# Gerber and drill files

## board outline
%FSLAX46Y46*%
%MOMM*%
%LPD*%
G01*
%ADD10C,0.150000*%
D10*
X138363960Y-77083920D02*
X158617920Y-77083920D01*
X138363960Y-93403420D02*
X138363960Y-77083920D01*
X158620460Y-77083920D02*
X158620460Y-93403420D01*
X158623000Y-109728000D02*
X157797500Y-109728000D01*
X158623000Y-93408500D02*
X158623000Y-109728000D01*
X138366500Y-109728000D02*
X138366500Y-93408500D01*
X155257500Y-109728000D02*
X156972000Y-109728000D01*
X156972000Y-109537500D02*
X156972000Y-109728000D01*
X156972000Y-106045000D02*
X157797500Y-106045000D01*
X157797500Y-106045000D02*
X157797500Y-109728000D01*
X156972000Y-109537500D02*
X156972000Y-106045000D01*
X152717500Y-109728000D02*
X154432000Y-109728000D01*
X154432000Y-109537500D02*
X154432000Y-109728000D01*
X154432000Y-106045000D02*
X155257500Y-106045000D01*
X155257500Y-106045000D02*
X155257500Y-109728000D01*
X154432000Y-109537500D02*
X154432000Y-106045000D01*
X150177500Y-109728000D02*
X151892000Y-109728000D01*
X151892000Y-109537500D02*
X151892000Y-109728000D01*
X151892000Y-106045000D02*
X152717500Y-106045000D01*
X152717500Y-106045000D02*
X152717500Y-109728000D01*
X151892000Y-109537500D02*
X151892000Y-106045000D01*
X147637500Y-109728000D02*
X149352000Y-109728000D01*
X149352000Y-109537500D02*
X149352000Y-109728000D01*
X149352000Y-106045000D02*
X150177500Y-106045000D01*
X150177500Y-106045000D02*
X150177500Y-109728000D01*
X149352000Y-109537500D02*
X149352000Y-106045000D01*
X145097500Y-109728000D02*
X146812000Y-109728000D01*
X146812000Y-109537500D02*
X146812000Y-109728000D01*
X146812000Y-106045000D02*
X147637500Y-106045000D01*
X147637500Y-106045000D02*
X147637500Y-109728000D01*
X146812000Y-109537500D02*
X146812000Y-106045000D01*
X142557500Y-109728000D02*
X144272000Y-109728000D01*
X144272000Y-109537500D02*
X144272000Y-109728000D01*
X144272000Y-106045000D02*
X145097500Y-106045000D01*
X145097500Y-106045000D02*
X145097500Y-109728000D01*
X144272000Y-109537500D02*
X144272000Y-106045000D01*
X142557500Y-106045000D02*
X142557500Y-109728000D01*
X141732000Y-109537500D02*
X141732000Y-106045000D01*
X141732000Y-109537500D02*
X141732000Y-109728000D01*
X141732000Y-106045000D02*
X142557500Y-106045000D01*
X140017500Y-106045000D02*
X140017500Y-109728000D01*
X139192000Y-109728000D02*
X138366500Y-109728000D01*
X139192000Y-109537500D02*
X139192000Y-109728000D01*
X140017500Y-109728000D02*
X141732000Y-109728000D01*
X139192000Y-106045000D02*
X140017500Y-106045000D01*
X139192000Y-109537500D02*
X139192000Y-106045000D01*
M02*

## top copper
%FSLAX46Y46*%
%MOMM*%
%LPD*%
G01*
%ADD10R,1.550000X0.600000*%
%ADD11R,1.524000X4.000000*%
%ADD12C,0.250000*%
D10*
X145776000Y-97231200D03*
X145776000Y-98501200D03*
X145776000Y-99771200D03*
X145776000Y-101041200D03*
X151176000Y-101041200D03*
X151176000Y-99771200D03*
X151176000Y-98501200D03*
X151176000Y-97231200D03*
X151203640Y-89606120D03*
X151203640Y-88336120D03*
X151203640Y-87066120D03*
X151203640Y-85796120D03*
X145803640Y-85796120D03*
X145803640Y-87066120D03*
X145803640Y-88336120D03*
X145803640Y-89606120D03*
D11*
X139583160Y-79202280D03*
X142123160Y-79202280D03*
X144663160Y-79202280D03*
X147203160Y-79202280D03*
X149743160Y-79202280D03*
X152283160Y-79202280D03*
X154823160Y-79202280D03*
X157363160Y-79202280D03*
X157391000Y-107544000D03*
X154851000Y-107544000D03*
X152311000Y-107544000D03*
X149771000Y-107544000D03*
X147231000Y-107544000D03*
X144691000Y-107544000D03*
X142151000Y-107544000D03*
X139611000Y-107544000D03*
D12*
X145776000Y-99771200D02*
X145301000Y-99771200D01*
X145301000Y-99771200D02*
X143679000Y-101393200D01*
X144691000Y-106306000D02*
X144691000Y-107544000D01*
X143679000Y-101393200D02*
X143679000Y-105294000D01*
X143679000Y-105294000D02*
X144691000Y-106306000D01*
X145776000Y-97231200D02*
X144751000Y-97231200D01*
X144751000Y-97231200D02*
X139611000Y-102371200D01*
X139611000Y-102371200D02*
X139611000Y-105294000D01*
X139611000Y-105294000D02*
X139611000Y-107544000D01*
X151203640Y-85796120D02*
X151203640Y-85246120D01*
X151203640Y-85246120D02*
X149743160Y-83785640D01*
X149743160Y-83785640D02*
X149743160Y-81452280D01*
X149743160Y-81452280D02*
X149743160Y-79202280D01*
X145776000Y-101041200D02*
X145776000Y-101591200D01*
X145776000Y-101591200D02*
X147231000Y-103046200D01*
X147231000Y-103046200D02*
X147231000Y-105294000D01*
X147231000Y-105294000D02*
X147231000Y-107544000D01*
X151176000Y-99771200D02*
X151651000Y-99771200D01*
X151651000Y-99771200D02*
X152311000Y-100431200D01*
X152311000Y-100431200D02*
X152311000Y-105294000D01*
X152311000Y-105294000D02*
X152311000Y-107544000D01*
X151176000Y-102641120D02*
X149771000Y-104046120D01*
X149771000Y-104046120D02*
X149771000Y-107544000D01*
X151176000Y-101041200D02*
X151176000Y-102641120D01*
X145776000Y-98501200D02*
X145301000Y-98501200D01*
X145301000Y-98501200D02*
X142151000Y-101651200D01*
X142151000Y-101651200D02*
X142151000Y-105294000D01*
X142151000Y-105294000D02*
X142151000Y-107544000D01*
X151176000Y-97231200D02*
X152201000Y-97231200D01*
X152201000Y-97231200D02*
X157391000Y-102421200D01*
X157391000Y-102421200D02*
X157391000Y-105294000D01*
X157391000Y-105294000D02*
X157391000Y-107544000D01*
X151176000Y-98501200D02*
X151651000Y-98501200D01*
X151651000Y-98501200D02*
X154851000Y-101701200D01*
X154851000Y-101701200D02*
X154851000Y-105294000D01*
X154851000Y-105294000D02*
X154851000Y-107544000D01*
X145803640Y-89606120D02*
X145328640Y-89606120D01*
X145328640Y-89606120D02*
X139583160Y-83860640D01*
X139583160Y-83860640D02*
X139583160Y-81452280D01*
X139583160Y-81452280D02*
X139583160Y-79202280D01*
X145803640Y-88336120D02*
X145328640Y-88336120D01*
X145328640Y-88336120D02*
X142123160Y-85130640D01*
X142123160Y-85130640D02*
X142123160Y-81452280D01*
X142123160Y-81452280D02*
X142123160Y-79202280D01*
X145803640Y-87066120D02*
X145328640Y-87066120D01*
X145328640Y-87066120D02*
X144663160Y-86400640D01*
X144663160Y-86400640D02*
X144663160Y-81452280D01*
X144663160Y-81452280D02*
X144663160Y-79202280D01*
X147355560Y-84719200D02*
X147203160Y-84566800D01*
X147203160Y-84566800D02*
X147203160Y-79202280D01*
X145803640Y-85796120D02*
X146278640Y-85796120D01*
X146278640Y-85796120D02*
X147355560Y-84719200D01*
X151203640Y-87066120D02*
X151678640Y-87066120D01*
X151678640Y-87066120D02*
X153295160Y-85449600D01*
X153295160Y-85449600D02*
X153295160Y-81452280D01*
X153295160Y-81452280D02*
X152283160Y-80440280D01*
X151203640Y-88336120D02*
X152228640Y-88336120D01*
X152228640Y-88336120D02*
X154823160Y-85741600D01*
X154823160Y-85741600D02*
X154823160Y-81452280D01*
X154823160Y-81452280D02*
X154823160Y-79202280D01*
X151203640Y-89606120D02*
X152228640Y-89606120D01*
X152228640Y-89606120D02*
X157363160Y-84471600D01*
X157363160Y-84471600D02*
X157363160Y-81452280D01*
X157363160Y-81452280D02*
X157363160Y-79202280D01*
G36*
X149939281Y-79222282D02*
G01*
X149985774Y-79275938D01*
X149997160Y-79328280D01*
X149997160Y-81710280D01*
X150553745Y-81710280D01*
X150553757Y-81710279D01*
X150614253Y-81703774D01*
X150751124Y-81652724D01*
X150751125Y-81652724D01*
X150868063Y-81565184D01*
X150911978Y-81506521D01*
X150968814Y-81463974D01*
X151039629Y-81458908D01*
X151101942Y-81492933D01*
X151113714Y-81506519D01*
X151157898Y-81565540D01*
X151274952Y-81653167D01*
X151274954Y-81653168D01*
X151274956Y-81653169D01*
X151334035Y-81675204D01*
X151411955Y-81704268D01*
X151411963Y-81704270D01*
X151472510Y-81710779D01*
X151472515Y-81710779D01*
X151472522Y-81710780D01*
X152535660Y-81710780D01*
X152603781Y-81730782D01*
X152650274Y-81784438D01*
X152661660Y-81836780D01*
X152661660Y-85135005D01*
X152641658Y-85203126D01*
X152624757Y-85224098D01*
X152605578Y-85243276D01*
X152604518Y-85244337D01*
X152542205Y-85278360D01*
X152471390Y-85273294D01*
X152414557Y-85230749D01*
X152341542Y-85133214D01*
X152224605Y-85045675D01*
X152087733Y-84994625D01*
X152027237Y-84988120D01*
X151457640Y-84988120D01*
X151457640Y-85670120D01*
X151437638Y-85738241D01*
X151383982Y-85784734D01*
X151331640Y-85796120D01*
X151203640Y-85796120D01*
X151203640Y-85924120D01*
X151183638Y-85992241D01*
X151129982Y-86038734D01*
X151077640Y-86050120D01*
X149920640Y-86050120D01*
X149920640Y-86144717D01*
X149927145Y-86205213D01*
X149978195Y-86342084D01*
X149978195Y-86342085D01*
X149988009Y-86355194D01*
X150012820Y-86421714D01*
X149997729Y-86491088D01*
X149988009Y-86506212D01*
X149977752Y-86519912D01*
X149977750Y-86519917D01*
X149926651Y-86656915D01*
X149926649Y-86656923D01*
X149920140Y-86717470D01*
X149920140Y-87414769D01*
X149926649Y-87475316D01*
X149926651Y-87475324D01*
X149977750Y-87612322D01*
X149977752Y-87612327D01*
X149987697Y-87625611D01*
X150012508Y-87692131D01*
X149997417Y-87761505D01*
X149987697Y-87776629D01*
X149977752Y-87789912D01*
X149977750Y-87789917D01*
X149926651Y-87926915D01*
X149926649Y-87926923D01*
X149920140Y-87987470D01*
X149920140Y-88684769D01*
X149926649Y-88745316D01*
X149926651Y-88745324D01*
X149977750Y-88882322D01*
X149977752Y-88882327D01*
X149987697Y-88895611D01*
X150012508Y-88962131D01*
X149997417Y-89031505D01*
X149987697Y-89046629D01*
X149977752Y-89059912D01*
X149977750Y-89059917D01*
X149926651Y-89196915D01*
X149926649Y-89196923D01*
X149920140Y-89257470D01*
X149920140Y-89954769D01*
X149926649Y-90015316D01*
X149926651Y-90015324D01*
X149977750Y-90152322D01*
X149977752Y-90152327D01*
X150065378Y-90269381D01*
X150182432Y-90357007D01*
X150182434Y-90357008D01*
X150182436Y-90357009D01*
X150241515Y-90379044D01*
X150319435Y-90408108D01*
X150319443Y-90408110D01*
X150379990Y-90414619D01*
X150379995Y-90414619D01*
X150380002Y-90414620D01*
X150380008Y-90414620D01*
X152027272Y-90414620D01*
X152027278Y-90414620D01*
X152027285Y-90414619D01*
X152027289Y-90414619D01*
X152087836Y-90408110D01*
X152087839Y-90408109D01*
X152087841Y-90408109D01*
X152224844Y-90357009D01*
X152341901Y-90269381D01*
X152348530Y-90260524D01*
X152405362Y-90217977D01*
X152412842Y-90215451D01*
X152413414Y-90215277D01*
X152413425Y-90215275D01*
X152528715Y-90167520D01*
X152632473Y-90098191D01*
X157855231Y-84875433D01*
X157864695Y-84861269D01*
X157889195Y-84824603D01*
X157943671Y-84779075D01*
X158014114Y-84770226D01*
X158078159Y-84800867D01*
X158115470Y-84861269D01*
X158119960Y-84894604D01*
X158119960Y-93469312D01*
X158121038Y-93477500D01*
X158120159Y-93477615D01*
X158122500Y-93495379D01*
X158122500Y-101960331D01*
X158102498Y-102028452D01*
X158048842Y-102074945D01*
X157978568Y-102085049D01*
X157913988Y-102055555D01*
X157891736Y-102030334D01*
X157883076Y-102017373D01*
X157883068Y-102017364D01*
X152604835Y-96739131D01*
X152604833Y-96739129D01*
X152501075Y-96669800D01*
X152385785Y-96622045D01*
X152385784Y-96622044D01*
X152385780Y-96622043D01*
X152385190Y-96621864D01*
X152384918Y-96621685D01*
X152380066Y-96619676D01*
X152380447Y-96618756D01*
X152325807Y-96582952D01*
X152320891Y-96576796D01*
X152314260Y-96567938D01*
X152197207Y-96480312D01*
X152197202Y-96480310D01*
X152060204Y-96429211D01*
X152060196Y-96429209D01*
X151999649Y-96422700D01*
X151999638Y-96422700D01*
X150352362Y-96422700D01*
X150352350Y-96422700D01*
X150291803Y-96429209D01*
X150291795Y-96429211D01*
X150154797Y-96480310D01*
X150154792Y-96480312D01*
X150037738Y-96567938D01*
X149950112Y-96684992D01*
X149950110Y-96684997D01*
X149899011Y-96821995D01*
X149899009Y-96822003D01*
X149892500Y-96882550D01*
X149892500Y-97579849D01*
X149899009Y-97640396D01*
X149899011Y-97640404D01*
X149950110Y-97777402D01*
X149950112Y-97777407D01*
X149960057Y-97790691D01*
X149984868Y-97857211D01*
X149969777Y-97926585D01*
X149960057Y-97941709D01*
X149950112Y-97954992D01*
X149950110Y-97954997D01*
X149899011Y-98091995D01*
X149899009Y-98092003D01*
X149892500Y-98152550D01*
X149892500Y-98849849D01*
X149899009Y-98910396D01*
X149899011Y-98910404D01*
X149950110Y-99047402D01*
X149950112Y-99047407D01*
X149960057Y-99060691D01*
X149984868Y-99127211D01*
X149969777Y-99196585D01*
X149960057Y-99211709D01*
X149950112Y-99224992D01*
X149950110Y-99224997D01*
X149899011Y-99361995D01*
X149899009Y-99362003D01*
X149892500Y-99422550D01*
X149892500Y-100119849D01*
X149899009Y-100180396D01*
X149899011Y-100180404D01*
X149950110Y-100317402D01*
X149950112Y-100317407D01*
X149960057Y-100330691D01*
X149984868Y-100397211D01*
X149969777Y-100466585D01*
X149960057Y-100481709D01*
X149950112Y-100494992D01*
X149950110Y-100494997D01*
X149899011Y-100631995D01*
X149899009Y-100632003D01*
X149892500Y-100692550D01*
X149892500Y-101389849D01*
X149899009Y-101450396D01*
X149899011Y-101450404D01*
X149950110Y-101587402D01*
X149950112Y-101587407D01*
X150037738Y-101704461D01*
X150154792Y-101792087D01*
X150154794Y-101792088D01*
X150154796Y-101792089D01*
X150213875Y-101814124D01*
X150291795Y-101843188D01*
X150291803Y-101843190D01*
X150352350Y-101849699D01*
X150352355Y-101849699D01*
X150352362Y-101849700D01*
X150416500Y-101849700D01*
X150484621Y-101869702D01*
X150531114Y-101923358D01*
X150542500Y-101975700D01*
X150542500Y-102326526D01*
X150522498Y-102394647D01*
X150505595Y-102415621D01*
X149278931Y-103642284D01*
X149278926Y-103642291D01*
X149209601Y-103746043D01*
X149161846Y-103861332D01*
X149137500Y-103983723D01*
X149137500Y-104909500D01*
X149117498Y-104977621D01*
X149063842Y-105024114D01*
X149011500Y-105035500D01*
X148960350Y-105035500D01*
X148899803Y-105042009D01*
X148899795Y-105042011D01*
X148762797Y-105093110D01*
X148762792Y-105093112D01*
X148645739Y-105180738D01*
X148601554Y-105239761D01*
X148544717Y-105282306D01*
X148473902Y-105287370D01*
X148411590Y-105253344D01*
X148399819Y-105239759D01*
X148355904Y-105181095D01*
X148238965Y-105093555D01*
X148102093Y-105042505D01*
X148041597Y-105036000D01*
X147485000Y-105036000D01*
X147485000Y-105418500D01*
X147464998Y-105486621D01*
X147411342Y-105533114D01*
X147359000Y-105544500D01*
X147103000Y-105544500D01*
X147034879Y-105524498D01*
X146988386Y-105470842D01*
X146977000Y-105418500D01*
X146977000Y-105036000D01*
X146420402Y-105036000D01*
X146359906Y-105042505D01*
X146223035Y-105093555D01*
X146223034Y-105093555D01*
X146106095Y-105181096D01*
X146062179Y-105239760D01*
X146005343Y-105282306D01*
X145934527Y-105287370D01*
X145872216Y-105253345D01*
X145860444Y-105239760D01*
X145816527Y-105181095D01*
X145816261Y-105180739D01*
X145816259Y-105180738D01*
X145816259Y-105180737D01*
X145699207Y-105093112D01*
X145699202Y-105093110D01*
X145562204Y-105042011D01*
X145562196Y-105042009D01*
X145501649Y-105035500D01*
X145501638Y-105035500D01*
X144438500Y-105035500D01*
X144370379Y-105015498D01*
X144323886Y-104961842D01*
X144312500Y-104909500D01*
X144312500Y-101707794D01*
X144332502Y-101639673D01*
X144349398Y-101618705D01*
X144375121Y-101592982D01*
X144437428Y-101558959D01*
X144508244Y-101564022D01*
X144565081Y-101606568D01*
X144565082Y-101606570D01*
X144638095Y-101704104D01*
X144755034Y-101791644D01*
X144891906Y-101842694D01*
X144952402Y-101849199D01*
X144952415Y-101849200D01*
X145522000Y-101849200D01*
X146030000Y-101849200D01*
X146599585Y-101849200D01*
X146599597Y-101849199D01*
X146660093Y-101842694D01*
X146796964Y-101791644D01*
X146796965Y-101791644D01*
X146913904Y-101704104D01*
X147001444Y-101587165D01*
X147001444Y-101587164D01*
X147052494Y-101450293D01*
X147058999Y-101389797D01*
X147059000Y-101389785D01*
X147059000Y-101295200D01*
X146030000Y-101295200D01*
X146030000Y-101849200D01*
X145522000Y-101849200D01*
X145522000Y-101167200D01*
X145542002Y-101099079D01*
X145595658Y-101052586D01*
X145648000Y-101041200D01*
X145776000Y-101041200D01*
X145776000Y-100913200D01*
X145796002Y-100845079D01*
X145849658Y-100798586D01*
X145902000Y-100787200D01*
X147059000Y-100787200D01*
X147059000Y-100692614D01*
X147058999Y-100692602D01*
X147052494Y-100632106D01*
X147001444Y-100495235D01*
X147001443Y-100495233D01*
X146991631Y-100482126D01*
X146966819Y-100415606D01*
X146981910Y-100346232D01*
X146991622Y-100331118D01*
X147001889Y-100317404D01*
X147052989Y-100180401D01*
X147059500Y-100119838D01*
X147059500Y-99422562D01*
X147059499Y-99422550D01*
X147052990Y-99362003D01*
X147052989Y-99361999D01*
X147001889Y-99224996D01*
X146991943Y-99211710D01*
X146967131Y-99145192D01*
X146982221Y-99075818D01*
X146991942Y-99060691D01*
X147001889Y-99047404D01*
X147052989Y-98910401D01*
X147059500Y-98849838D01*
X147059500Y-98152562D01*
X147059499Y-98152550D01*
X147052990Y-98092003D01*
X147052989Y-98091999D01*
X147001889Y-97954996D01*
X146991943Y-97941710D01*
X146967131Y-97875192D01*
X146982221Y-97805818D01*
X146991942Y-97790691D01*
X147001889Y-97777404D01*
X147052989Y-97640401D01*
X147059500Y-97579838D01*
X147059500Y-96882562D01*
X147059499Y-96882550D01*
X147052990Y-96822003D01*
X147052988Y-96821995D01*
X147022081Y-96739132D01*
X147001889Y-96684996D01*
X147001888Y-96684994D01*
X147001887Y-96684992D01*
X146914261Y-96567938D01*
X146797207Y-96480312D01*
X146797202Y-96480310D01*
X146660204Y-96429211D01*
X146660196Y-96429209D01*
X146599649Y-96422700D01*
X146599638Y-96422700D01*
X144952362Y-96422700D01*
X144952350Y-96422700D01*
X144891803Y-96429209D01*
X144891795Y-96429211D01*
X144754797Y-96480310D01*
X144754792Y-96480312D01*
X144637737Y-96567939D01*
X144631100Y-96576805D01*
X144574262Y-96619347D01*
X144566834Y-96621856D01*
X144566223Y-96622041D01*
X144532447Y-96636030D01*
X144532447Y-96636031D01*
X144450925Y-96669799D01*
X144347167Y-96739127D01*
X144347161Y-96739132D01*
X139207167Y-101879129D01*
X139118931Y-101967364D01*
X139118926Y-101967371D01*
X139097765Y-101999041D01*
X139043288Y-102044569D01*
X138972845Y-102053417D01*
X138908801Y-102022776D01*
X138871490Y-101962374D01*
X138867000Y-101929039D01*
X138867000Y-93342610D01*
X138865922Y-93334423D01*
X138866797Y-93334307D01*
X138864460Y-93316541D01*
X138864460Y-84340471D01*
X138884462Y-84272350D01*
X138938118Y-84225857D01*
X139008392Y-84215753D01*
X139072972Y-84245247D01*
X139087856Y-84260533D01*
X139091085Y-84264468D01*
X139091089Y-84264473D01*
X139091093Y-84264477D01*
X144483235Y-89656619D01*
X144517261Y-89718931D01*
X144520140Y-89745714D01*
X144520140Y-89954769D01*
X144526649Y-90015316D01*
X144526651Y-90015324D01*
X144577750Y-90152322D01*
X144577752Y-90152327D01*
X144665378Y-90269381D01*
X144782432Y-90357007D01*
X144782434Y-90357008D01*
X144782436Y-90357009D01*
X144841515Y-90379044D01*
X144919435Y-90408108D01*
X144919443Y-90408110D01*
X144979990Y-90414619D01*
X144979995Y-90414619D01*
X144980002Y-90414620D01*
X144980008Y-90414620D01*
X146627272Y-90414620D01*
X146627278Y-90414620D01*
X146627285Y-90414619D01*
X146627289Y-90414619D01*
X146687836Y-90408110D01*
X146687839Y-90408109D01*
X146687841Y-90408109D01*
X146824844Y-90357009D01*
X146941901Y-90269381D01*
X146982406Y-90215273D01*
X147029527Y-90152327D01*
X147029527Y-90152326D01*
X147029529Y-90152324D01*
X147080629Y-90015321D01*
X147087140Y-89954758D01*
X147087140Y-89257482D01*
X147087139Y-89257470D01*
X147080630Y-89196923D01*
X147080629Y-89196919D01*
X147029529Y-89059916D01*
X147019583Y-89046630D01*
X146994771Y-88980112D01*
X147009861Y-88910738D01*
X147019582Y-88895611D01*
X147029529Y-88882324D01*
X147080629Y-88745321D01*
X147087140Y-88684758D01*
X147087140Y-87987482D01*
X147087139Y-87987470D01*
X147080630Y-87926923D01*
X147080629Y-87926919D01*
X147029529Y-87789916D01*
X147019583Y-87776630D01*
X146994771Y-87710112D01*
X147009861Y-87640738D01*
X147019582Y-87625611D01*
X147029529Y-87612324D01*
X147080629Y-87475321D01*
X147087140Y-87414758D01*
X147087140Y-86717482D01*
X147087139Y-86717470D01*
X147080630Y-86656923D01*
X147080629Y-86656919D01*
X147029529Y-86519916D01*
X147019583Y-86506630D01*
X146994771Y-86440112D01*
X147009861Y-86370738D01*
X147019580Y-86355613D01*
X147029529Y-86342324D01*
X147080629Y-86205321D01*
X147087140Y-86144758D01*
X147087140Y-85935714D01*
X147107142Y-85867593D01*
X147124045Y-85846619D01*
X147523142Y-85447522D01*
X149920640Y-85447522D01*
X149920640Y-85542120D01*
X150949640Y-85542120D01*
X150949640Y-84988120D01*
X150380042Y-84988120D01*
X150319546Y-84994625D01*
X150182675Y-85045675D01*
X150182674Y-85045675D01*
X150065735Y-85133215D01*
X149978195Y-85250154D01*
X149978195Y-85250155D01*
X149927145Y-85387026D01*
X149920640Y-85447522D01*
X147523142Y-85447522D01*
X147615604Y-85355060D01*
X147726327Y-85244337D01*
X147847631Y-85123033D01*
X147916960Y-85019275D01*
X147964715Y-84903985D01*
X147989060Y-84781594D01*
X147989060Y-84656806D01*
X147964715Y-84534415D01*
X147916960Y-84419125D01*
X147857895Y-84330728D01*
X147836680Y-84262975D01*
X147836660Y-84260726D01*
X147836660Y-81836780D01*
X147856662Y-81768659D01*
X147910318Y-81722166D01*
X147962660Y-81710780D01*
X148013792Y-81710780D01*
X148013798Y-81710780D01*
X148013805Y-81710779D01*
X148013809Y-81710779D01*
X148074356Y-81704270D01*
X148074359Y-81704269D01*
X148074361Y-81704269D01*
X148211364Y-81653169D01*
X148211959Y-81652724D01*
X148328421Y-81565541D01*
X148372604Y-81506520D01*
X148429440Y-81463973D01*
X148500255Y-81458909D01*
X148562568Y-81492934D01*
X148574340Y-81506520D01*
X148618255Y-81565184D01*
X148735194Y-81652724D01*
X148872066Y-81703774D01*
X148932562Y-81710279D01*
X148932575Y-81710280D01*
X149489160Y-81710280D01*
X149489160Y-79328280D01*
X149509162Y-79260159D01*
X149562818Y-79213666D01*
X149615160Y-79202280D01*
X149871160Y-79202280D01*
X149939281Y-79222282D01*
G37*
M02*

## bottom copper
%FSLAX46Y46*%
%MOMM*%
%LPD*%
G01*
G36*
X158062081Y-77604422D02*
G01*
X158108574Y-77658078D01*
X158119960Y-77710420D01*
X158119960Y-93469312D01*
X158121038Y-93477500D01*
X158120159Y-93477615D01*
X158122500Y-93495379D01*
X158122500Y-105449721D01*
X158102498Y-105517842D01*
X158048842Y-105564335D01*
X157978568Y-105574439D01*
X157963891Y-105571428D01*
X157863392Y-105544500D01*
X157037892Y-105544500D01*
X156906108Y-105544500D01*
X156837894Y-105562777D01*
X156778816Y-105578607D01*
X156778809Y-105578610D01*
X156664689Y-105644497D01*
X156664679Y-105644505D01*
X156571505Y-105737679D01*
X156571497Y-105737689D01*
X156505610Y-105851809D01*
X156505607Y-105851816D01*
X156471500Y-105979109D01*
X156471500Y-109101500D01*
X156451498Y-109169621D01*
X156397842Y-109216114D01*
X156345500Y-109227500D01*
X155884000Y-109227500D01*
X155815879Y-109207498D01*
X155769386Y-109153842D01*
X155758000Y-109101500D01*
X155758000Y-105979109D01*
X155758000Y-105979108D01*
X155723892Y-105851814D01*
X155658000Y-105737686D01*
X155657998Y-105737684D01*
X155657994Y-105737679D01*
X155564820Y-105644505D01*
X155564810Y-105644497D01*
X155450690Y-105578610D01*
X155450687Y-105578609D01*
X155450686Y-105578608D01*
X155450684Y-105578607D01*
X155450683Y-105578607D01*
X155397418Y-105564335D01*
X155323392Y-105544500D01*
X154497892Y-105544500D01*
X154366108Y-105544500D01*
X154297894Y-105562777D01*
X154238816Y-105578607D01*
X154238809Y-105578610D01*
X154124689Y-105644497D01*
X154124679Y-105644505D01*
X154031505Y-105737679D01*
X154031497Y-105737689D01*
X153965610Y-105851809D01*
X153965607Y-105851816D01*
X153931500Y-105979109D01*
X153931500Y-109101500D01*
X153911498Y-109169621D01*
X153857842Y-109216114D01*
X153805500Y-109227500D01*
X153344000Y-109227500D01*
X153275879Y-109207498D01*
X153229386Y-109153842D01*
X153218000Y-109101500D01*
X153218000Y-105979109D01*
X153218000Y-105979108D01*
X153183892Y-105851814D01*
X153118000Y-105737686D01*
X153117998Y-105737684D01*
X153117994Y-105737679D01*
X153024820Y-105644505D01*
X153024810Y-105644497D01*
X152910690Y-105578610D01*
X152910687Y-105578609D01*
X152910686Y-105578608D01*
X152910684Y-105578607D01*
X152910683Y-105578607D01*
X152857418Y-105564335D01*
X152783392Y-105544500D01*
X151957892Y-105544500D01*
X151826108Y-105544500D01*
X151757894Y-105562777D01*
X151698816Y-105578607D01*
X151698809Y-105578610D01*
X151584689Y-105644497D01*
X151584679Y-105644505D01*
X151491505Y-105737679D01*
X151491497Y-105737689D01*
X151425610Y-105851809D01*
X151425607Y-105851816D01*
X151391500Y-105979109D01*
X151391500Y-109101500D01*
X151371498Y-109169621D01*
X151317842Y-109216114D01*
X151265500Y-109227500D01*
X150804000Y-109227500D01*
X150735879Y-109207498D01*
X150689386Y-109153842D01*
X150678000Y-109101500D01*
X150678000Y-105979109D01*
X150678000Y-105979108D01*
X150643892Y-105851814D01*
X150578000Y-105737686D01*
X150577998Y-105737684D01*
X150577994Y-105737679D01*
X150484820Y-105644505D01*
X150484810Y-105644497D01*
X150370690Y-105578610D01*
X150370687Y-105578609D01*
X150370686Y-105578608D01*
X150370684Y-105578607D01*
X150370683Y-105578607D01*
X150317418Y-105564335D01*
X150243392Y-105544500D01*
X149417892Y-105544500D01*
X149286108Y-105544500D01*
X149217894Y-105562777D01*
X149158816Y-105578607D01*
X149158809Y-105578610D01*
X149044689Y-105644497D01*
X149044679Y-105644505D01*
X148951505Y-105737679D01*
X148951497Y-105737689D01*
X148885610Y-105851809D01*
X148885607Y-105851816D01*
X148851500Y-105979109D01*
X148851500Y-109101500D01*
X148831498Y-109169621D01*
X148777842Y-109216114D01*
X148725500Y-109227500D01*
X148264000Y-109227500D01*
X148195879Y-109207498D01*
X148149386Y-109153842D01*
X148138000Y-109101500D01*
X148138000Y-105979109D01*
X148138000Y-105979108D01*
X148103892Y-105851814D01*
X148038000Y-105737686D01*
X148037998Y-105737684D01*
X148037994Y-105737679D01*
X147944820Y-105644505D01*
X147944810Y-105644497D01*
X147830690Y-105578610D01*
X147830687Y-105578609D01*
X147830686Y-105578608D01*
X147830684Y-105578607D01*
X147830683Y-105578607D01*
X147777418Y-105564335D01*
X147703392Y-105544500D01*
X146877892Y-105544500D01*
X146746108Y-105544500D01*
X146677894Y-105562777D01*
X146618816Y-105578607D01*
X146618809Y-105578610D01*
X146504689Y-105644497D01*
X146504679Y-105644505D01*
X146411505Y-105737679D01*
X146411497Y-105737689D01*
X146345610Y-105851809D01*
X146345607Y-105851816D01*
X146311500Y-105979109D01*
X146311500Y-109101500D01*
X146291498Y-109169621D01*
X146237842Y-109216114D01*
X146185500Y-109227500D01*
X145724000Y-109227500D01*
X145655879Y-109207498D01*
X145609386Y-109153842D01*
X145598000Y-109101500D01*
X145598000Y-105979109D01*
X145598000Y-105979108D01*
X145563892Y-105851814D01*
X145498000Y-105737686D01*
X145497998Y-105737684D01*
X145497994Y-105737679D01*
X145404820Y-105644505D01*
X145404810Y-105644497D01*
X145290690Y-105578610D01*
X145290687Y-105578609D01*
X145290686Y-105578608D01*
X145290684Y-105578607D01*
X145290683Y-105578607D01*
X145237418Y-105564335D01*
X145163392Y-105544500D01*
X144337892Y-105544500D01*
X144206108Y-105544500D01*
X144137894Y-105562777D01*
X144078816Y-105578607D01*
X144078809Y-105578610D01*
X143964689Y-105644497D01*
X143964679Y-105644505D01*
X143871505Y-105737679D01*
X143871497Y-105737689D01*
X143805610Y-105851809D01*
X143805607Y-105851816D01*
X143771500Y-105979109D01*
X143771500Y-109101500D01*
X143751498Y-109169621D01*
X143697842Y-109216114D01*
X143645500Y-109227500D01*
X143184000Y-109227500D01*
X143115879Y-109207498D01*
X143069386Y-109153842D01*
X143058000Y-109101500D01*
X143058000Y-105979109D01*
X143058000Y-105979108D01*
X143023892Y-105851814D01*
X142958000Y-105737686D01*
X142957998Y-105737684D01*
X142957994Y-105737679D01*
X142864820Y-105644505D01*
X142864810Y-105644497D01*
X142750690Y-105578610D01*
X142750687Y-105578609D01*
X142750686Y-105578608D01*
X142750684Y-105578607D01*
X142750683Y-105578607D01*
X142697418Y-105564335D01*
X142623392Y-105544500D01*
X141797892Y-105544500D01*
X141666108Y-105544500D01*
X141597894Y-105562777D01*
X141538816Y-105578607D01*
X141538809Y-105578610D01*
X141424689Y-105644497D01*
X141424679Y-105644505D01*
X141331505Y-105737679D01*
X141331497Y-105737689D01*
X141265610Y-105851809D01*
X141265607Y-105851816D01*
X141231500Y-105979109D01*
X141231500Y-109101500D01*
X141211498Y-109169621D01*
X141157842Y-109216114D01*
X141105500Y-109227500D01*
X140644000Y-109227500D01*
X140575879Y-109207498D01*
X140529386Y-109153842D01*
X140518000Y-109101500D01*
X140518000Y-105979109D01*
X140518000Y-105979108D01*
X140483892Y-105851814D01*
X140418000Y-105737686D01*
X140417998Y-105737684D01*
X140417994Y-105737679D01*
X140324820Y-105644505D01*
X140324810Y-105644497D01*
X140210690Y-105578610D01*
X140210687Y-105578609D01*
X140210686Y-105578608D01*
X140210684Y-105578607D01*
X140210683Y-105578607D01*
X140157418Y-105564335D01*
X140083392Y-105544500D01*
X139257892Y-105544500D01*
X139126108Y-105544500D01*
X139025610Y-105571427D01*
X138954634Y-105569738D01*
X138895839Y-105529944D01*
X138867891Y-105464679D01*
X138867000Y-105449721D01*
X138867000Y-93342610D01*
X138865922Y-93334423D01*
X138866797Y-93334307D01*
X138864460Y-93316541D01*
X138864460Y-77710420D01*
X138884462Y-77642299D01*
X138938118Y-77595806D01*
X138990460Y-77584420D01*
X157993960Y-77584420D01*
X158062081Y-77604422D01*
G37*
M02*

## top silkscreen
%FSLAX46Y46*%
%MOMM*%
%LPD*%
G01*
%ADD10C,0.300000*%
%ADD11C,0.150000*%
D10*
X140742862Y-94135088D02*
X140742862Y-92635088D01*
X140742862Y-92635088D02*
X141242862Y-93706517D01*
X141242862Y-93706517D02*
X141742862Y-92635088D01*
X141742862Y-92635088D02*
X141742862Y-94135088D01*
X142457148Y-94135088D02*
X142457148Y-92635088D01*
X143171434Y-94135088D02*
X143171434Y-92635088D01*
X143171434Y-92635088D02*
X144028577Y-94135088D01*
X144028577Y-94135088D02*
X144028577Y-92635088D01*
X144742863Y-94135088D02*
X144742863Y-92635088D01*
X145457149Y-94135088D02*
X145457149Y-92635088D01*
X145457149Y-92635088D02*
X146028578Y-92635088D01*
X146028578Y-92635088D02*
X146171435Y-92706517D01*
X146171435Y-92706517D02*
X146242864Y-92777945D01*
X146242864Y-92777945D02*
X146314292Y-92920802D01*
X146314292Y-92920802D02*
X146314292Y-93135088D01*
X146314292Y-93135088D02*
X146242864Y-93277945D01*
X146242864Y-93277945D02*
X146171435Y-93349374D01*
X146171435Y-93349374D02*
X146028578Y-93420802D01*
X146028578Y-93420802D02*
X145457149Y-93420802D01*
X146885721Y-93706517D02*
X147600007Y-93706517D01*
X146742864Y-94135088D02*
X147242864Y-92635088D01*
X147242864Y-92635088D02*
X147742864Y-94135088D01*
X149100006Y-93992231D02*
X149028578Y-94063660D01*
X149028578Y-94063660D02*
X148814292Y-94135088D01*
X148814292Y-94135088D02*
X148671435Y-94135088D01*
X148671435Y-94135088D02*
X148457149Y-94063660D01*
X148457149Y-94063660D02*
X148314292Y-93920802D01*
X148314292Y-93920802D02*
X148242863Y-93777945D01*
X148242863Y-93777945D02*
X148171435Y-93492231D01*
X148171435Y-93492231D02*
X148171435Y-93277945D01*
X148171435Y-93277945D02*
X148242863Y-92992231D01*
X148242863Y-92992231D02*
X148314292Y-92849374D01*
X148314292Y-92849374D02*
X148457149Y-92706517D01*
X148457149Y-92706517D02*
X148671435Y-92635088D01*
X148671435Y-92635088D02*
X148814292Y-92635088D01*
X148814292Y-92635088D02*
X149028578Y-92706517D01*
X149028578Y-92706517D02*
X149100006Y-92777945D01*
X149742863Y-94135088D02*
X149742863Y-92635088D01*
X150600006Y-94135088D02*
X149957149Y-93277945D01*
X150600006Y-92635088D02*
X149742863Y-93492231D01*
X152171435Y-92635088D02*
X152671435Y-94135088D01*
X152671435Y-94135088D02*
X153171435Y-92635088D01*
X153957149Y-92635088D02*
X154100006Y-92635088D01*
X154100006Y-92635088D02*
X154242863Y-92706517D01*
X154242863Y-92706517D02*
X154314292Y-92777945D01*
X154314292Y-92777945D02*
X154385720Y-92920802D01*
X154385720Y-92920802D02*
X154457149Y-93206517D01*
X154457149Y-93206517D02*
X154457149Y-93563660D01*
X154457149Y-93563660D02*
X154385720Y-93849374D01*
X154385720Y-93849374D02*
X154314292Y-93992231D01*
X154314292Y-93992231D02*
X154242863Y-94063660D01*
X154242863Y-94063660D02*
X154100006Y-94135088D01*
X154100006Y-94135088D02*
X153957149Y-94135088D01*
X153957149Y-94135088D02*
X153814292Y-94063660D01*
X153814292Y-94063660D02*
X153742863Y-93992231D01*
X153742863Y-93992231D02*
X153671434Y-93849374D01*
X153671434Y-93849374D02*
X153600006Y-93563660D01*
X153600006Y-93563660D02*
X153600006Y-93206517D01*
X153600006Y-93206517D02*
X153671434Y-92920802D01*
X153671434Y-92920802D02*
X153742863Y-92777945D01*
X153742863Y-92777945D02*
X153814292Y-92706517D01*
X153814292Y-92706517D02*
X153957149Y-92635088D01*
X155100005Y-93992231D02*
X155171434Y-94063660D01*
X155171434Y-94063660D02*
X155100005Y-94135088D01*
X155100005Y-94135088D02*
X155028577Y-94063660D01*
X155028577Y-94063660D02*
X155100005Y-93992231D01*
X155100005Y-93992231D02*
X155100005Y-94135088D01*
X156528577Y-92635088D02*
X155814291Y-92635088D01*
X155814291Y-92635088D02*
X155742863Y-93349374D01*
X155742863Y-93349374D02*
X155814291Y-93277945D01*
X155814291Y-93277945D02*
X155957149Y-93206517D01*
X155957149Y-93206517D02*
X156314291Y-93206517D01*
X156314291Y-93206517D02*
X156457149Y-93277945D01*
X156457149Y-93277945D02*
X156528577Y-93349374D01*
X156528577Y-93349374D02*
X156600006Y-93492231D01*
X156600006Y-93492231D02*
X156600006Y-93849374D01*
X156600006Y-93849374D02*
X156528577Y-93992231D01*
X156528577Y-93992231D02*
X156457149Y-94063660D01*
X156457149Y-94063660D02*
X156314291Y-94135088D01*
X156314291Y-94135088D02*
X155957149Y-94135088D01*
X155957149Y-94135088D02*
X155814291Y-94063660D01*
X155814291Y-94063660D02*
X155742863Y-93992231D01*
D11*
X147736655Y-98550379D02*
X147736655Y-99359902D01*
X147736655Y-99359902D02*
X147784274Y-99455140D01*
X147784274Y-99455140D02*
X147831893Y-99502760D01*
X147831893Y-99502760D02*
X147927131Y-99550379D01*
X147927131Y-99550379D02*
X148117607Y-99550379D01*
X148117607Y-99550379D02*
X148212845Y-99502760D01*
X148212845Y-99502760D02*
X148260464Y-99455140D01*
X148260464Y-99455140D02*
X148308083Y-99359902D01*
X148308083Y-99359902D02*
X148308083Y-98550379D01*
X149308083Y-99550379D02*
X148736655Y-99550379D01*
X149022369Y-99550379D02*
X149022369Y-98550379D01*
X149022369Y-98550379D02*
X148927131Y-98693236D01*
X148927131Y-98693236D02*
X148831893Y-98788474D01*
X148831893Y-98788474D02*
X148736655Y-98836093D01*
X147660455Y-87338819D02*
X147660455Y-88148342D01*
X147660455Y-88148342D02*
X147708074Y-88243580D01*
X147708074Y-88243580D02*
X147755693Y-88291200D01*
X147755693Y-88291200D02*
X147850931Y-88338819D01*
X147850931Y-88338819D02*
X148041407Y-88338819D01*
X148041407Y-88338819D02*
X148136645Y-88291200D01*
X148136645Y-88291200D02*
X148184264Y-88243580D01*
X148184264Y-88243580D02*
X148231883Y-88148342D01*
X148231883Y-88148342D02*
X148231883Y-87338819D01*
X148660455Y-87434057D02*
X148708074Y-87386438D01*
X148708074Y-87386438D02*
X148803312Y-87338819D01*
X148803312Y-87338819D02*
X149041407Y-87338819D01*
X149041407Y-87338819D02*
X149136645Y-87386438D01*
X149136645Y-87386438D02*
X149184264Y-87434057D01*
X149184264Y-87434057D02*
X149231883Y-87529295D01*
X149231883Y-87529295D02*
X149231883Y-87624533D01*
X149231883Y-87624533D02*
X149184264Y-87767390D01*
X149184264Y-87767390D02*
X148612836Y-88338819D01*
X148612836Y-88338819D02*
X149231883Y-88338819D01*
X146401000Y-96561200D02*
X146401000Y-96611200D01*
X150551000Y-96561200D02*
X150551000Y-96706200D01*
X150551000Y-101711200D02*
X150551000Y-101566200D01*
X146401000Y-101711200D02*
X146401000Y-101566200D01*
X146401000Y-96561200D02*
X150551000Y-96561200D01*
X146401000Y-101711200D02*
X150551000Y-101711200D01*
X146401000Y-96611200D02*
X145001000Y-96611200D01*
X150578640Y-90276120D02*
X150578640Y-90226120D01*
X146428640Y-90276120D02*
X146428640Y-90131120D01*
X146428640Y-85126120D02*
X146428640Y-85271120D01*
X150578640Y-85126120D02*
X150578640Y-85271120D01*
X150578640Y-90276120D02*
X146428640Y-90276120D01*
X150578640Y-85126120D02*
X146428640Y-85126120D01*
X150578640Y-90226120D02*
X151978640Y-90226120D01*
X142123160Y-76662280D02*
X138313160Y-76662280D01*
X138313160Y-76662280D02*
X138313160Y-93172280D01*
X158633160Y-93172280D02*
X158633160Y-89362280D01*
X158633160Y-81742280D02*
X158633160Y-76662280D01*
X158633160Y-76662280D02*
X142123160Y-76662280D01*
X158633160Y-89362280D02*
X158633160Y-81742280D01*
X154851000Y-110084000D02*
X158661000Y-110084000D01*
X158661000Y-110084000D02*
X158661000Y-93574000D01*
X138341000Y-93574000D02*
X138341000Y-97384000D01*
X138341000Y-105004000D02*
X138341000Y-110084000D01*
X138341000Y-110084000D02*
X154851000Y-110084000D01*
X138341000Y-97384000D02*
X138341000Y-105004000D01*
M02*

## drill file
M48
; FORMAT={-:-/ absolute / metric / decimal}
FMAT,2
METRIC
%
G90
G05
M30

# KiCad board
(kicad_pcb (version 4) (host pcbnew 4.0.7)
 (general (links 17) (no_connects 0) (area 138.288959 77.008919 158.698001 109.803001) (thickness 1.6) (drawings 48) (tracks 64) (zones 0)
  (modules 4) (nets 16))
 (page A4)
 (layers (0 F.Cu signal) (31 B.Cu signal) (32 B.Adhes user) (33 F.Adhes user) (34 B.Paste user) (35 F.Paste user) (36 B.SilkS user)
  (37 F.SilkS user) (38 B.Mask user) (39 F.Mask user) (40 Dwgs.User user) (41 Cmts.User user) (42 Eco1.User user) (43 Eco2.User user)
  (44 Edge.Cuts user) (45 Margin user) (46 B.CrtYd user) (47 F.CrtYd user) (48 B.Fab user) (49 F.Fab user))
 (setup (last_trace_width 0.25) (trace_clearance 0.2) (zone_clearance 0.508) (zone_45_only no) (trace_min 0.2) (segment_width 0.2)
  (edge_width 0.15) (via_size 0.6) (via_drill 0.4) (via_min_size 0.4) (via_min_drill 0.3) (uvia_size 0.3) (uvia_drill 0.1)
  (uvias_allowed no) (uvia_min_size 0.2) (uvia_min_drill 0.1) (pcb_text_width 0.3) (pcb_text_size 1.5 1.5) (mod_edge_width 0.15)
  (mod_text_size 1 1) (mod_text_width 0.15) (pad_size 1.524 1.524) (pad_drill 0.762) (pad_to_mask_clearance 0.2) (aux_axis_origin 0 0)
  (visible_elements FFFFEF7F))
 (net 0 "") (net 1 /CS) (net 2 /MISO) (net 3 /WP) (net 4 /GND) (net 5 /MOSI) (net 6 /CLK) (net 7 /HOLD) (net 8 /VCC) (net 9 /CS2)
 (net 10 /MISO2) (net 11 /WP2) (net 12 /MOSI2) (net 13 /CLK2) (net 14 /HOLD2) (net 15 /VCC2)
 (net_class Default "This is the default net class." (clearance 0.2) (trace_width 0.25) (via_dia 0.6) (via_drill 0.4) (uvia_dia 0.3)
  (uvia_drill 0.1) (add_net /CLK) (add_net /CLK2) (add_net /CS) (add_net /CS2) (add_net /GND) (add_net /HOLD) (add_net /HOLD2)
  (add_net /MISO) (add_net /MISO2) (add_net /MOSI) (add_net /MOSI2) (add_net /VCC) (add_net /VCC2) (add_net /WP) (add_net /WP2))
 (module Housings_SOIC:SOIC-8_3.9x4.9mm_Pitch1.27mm (layer F.Cu) (at 148.476 99.1362)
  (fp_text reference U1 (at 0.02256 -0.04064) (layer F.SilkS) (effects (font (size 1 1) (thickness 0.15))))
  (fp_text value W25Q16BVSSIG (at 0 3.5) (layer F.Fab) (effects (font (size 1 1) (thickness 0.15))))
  (fp_line (start -2.075 -2.575) (end -2.075 -2.525) (layer F.SilkS) (width 0.15))
  (fp_line (start 2.075 -2.575) (end 2.075 -2.43) (layer F.SilkS) (width 0.15))
  (fp_line (start 2.075 2.575) (end 2.075 2.43) (layer F.SilkS) (width 0.15))
  (fp_line (start -2.075 2.575) (end -2.075 2.43) (layer F.SilkS) (width 0.15))
  (fp_line (start -2.075 -2.575) (end 2.075 -2.575) (layer F.SilkS) (width 0.15))
  (fp_line (start -2.075 2.575) (end 2.075 2.575) (layer F.SilkS) (width 0.15))
  (fp_line (start -2.075 -2.525) (end -3.475 -2.525) (layer F.SilkS) (width 0.15))
  (pad 1 smd rect (at -2.7 -1.905) (size 1.55 0.6) (layers F.Cu F.Paste F.Mask) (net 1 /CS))
  (pad 2 smd rect (at -2.7 -0.635) (size 1.55 0.6) (layers F.Cu F.Paste F.Mask) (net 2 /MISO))
  (pad 3 smd rect (at -2.7 0.635) (size 1.55 0.6) (layers F.Cu F.Paste F.Mask) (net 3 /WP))
  (pad 4 smd rect (at -2.7 1.905) (size 1.55 0.6) (layers F.Cu F.Paste F.Mask) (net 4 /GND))
  (pad 5 smd rect (at 2.7 1.905) (size 1.55 0.6) (layers F.Cu F.Paste F.Mask) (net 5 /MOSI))
  (pad 6 smd rect (at 2.7 0.635) (size 1.55 0.6) (layers F.Cu F.Paste F.Mask) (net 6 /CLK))
  (pad 7 smd rect (at 2.7 -0.635) (size 1.55 0.6) (layers F.Cu F.Paste F.Mask) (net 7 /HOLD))
  (pad 8 smd rect (at 2.7 -1.905) (size 1.55 0.6) (layers F.Cu F.Paste F.Mask) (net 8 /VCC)))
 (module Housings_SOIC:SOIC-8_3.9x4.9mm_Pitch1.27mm (layer F.Cu) (at 148.50364 87.70112 180)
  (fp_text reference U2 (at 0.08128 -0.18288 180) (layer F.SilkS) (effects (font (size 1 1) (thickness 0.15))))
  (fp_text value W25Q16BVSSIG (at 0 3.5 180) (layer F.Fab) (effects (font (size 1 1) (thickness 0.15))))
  (fp_line (start -2.075 -2.575) (end -2.075 -2.525) (layer F.SilkS) (width 0.15))
  (fp_line (start 2.075 -2.575) (end 2.075 -2.43) (layer F.SilkS) (width 0.15))
  (fp_line (start 2.075 2.575) (end 2.075 2.43) (layer F.SilkS) (width 0.15))
  (fp_line (start -2.075 2.575) (end -2.075 2.43) (layer F.SilkS) (width 0.15))
  (fp_line (start -2.075 -2.575) (end 2.075 -2.575) (layer F.SilkS) (width 0.15))
  (fp_line (start -2.075 2.575) (end 2.075 2.575) (layer F.SilkS) (width 0.15))
  (fp_line (start -2.075 -2.525) (end -3.475 -2.525) (layer F.SilkS) (width 0.15))
  (pad 1 smd rect (at -2.7 -1.905 180) (size 1.55 0.6) (layers F.Cu F.Paste F.Mask) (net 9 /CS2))
  (pad 2 smd rect (at -2.7 -0.635 180) (size 1.55 0.6) (layers F.Cu F.Paste F.Mask) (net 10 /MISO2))
  (pad 3 smd rect (at -2.7 0.635 180) (size 1.55 0.6) (layers F.Cu F.Paste F.Mask) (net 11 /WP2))
  (pad 4 smd rect (at -2.7 1.905 180) (size 1.55 0.6) (layers F.Cu F.Paste F.Mask) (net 4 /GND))
  (pad 5 smd rect (at 2.7 1.905 180) (size 1.55 0.6) (layers F.Cu F.Paste F.Mask) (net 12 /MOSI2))
  (pad 6 smd rect (at 2.7 0.635 180) (size 1.55 0.6) (layers F.Cu F.Paste F.Mask) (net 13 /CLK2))
  (pad 7 smd rect (at 2.7 -0.635 180) (size 1.55 0.6) (layers F.Cu F.Paste F.Mask) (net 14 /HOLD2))
  (pad 8 smd rect (at 2.7 -1.905 180) (size 1.55 0.6) (layers F.Cu F.Paste F.Mask) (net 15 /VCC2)))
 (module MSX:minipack (layer F.Cu) (at 148.47316 81.74228 180)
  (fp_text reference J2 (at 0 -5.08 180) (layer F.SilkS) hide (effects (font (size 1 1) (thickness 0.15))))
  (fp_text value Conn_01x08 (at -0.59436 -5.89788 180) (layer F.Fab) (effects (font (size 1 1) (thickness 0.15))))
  (fp_line (start 6.35 5.08) (end 10.16 5.08) (layer F.SilkS) (width 0.15))
  (fp_line (start 10.16 5.08) (end 10.16 -11.43) (layer F.SilkS) (width 0.15))
  (fp_line (start -10.16 -11.43) (end -10.16 -7.62) (layer F.SilkS) (width 0.15))
  (fp_line (start -10.16 0) (end -10.16 5.08) (layer F.SilkS) (width 0.15))
  (fp_line (start -10.16 5.08) (end 6.35 5.08) (layer F.SilkS) (width 0.15))
  (fp_line (start -10.16 -7.62) (end -10.16 0) (layer F.SilkS) (width 0.15))
  (pad 8 smd rect (at 8.89 2.54 180) (size 1.524 4) (layers F.Cu F.Paste F.Mask) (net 15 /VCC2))
  (pad 7 smd rect (at 6.35 2.54 180) (size 1.524 4) (layers F.Cu F.Paste F.Mask) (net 14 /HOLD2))
  (pad 6 smd rect (at 3.81 2.54 180) (size 1.524 4) (layers F.Cu F.Paste F.Mask) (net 13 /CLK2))
  (pad 5 smd rect (at 1.27 2.54 180) (size 1.524 4) (layers F.Cu F.Paste F.Mask) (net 12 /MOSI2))
  (pad 4 smd rect (at -1.27 2.54 180) (size 1.524 4) (layers F.Cu F.Paste F.Mask) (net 4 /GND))
  (pad 3 smd rect (at -3.81 2.54 180) (size 1.524 4) (layers F.Cu F.Paste F.Mask) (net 11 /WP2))
  (pad 2 smd rect (at -6.35 2.54 180) (size 1.524 4) (layers F.Cu F.Paste F.Mask) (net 10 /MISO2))
  (pad 1 smd rect (at -8.89 2.54 180) (size 1.524 4) (layers F.Cu F.Paste F.Mask) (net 9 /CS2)))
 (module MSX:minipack (layer F.Cu) (at 148.501 105.004)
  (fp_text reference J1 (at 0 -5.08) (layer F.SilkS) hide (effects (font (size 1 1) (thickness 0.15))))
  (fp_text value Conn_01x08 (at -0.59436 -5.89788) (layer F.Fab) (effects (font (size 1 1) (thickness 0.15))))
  (fp_line (start 6.35 5.08) (end 10.16 5.08) (layer F.SilkS) (width 0.15))
  (fp_line (start 10.16 5.08) (end 10.16 -11.43) (layer F.SilkS) (width 0.15))
  (fp_line (start -10.16 -11.43) (end -10.16 -7.62) (layer F.SilkS) (width 0.15))
  (fp_line (start -10.16 0) (end -10.16 5.08) (layer F.SilkS) (width 0.15))
  (fp_line (start -10.16 5.08) (end 6.35 5.08) (layer F.SilkS) (width 0.15))
  (fp_line (start -10.16 -7.62) (end -10.16 0) (layer F.SilkS) (width 0.15))
  (pad 8 smd rect (at 8.89 2.54) (size 1.524 4) (layers F.Cu F.Paste F.Mask) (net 8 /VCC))
  (pad 7 smd rect (at 6.35 2.54) (size 1.524 4) (layers F.Cu F.Paste F.Mask) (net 7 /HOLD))
  (pad 6 smd rect (at 3.81 2.54) (size 1.524 4) (layers F.Cu F.Paste F.Mask) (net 6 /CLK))
  (pad 5 smd rect (at 1.27 2.54) (size 1.524 4) (layers F.Cu F.Paste F.Mask) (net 5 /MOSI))
  (pad 4 smd rect (at -1.27 2.54) (size 1.524 4) (layers F.Cu F.Paste F.Mask) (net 4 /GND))
  (pad 3 smd rect (at -3.81 2.54) (size 1.524 4) (layers F.Cu F.Paste F.Mask) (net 3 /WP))
  (pad 2 smd rect (at -6.35 2.54) (size 1.524 4) (layers F.Cu F.Paste F.Mask) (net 2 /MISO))
  (pad 1 smd rect (at -8.89 2.54) (size 1.524 4) (layers F.Cu F.Paste F.Mask) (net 1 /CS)))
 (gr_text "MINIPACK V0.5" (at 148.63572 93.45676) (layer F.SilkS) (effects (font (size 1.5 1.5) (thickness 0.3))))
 (gr_line (start 138.36396 77.08392) (end 158.61792 77.08392) (layer Edge.Cuts) (width 0.15))
 (gr_line (start 138.36396 93.40342) (end 138.36396 77.08392) (layer Edge.Cuts) (width 0.15))
 (gr_line (start 158.62046 77.08392) (end 158.62046 93.40342) (layer Edge.Cuts) (width 0.15))
 (gr_line (start 158.623 109.728) (end 157.7975 109.728) (layer Edge.Cuts) (width 0.15))
 (gr_line (start 158.623 93.4085) (end 158.623 109.728) (layer Edge.Cuts) (width 0.15))
 (gr_line (start 138.3665 109.728) (end 138.3665 93.4085) (layer Edge.Cuts) (width 0.15))
 (gr_line (start 155.2575 109.728) (end 156.972 109.728) (layer Edge.Cuts) (width 0.15))
 (gr_line (start 156.972 109.5375) (end 156.972 109.728) (layer Edge.Cuts) (width 0.15))
 (gr_line (start 156.972 106.045) (end 157.7975 106.045) (layer Edge.Cuts) (width 0.15))
 (gr_line (start 157.7975 106.045) (end 157.7975 109.728) (layer Edge.Cuts) (width 0.15))
 (gr_line (start 156.972 109.5375) (end 156.972 106.045) (layer Edge.Cuts) (width 0.15))
 (gr_line (start 152.7175 109.728) (end 154.432 109.728) (layer Edge.Cuts) (width 0.15))
 (gr_line (start 154.432 109.5375) (end 154.432 109.728) (layer Edge.Cuts) (width 0.15))
 (gr_line (start 154.432 106.045) (end 155.2575 106.045) (layer Edge.Cuts) (width 0.15))
 (gr_line (start 155.2575 106.045) (end 155.2575 109.728) (layer Edge.Cuts) (width 0.15))
 (gr_line (start 154.432 109.5375) (end 154.432 106.045) (layer Edge.Cuts) (width 0.15))
 (gr_line (start 150.1775 109.728) (end 151.892 109.728) (layer Edge.Cuts) (width 0.15))
 (gr_line (start 151.892 109.5375) (end 151.892 109.728) (layer Edge.Cuts) (width 0.15))
 (gr_line (start 151.892 106.045) (end 152.7175 106.045) (layer Edge.Cuts) (width 0.15))
 (gr_line (start 152.7175 106.045) (end 152.7175 109.728) (layer Edge.Cuts) (width 0.15))
 (gr_line (start 151.892 109.5375) (end 151.892 106.045) (layer Edge.Cuts) (width 0.15))
 (gr_line (start 147.6375 109.728) (end 149.352 109.728) (layer Edge.Cuts) (width 0.15))
 (gr_line (start 149.352 109.5375) (end 149.352 109.728) (layer Edge.Cuts) (width 0.15))
 (gr_line (start 149.352 106.045) (end 150.1775 106.045) (layer Edge.Cuts) (width 0.15))
 (gr_line (start 150.1775 106.045) (end 150.1775 109.728) (layer Edge.Cuts) (width 0.15))
 (gr_line (start 149.352 109.5375) (end 149.352 106.045) (layer Edge.Cuts) (width 0.15))
 (gr_line (start 145.0975 109.728) (end 146.812 109.728) (layer Edge.Cuts) (width 0.15))
 (gr_line (start 146.812 109.5375) (end 146.812 109.728) (layer Edge.Cuts) (width 0.15))
 (gr_line (start 146.812 106.045) (end 147.6375 106.045) (layer Edge.Cuts) (width 0.15))
 (gr_line (start 147.6375 106.045) (end 147.6375 109.728) (layer Edge.Cuts) (width 0.15))
 (gr_line (start 146.812 109.5375) (end 146.812 106.045) (layer Edge.Cuts) (width 0.15))
 (gr_line (start 142.5575 109.728) (end 144.272 109.728) (layer Edge.Cuts) (width 0.15))
 (gr_line (start 144.272 109.5375) (end 144.272 109.728) (layer Edge.Cuts) (width 0.15))
 (gr_line (start 144.272 106.045) (end 145.0975 106.045) (layer Edge.Cuts) (width 0.15))
 (gr_line (start 145.0975 106.045) (end 145.0975 109.728) (layer Edge.Cuts) (width 0.15))
 (gr_line (start 144.272 109.5375) (end 144.272 106.045) (layer Edge.Cuts) (width 0.15))
 (gr_line (start 142.5575 106.045) (end 142.5575 109.728) (layer Edge.Cuts) (width 0.15))
 (gr_line (start 141.732 109.5375) (end 141.732 106.045) (layer Edge.Cuts) (width 0.15))
 (gr_line (start 141.732 109.5375) (end 141.732 109.728) (layer Edge.Cuts) (width 0.15))
 (gr_line (start 141.732 106.045) (end 142.5575 106.045) (layer Edge.Cuts) (width 0.15))
 (gr_line (start 140.0175 106.045) (end 140.0175 109.728) (layer Edge.Cuts) (width 0.15))
 (gr_line (start 139.192 109.728) (end 138.3665 109.728) (layer Edge.Cuts) (width 0.15))
 (gr_line (start 139.192 109.5375) (end 139.192 109.728) (layer Edge.Cuts) (width 0.15))
 (gr_line (start 140.0175 109.728) (end 141.732 109.728) (layer Edge.Cuts) (width 0.15))
 (gr_line (start 139.192 106.045) (end 140.0175 106.045) (layer Edge.Cuts) (width 0.15))
 (gr_line (start 139.192 109.5375) (end 139.192 106.045) (layer Edge.Cuts) (width 0.15))
 (segment (start 145.776 99.7712) (end 145.301 99.7712) (width 0.25) (layer F.Cu) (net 3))
 (segment (start 145.301 99.7712) (end 143.679 101.3932) (width 0.25) (layer F.Cu) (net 3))
 (segment (start 144.691 106.306) (end 144.691 107.544) (width 0.25) (layer F.Cu) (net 3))
 (segment (start 143.679 101.3932) (end 143.679 105.294) (width 0.25) (layer F.Cu) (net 3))
 (segment (start 143.679 105.294) (end 144.691 106.306) (width 0.25) (layer F.Cu) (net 3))
 (segment (start 145.776 97.2312) (end 144.751 97.2312) (width 0.25) (layer F.Cu) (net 1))
 (segment (start 144.751 97.2312) (end 139.611 102.3712) (width 0.25) (layer F.Cu) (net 1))
 (segment (start 139.611 102.3712) (end 139.611 105.294) (width 0.25) (layer F.Cu) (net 1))
 (segment (start 139.611 105.294) (end 139.611 107.544) (width 0.25) (layer F.Cu) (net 1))
 (segment (start 151.20364 85.79612) (end 151.20364 85.24612) (width 0.25) (layer F.Cu) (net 4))
 (segment (start 151.20364 85.24612) (end 149.74316 83.78564) (width 0.25) (layer F.Cu) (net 4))
 (segment (start 149.74316 83.78564) (end 149.74316 81.45228) (width 0.25) (layer F.Cu) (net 4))
 (segment (start 149.74316 81.45228) (end 149.74316 79.20228) (width 0.25) (layer F.Cu) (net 4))
 (segment (start 145.776 101.0412) (end 145.776 101.5912) (width 0.25) (layer F.Cu) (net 4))
 (segment (start 145.776 101.5912) (end 147.231 103.0462) (width 0.25) (layer F.Cu) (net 4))
 (segment (start 147.231 103.0462) (end 147.231 105.294) (width 0.25) (layer F.Cu) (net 4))
 (segment (start 147.231 105.294) (end 147.231 107.544) (width 0.25) (layer F.Cu) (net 4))
 (segment (start 151.176 99.7712) (end 151.651 99.7712) (width 0.25) (layer F.Cu) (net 6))
 (segment (start 151.651 99.7712) (end 152.311 100.4312) (width 0.25) (layer F.Cu) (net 6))
 (segment (start 152.311 100.4312) (end 152.311 105.294) (width 0.25) (layer F.Cu) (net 6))
 (segment (start 152.311 105.294) (end 152.311 107.544) (width 0.25) (layer F.Cu) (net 6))
 (segment (start 151.176 102.64112) (end 149.771 104.04612) (width 0.25) (layer F.Cu) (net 5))
 (segment (start 149.771 104.04612) (end 149.771 107.544) (width 0.25) (layer F.Cu) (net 5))
 (segment (start 151.176 101.0412) (end 151.176 102.64112) (width 0.25) (layer F.Cu) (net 5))
 (segment (start 145.776 98.5012) (end 145.301 98.5012) (width 0.25) (layer F.Cu) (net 2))
 (segment (start 145.301 98.5012) (end 142.151 101.6512) (width 0.25) (layer F.Cu) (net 2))
 (segment (start 142.151 101.6512) (end 142.151 105.294) (width 0.25) (layer F.Cu) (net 2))
 (segment (start 142.151 105.294) (end 142.151 107.544) (width 0.25) (layer F.Cu) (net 2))
 (segment (start 151.176 97.2312) (end 152.201 97.2312) (width 0.25) (layer F.Cu) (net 8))
 (segment (start 152.201 97.2312) (end 157.391 102.4212) (width 0.25) (layer F.Cu) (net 8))
 (segment (start 157.391 102.4212) (end 157.391 105.294) (width 0.25) (layer F.Cu) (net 8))
 (segment (start 157.391 105.294) (end 157.391 107.544) (width 0.25) (layer F.Cu) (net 8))
 (segment (start 151.176 98.5012) (end 151.651 98.5012) (width 0.25) (layer F.Cu) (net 7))
 (segment (start 151.651 98.5012) (end 154.851 101.7012) (width 0.25) (layer F.Cu) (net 7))
 (segment (start 154.851 101.7012) (end 154.851 105.294) (width 0.25) (layer F.Cu) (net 7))
 (segment (start 154.851 105.294) (end 154.851 107.544) (width 0.25) (layer F.Cu) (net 7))
 (segment (start 145.80364 89.60612) (end 145.32864 89.60612) (width 0.25) (layer F.Cu) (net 15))
 (segment (start 145.32864 89.60612) (end 139.58316 83.86064) (width 0.25) (layer F.Cu) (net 15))
 (segment (start 139.58316 83.86064) (end 139.58316 81.45228) (width 0.25) (layer F.Cu) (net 15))
 (segment (start 139.58316 81.45228) (end 139.58316 79.20228) (width 0.25) (layer F.Cu) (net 15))
 (segment (start 145.80364 88.33612) (end 145.32864 88.33612) (width 0.25) (layer F.Cu) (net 14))
 (segment (start 145.32864 88.33612) (end 142.12316 85.13064) (width 0.25) (layer F.Cu) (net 14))
 (segment (start 142.12316 85.13064) (end 142.12316 81.45228) (width 0.25) (layer F.Cu) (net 14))
 (segment (start 142.12316 81.45228) (end 142.12316 79.20228) (width 0.25) (layer F.Cu) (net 14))
 (segment (start 145.80364 87.06612) (end 145.32864 87.06612) (width 0.25) (layer F.Cu) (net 13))
 (segment (start 145.32864 87.06612) (end 144.66316 86.40064) (width 0.25) (layer F.Cu) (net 13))
 (segment (start 144.66316 86.40064) (end 144.66316 81.45228) (width 0.25) (layer F.Cu) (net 13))
 (segment (start 144.66316 81.45228) (end 144.66316 79.20228) (width 0.25) (layer F.Cu) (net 13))
 (segment (start 147.35556 84.7192) (end 147.20316 84.5668) (width 0.25) (layer F.Cu) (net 12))
 (segment (start 147.20316 84.5668) (end 147.20316 79.20228) (width 0.25) (layer F.Cu) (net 12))
 (segment (start 145.80364 85.79612) (end 146.27864 85.79612) (width 0.25) (layer F.Cu) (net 12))
 (segment (start 146.27864 85.79612) (end 147.35556 84.7192) (width 0.25) (layer F.Cu) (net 12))
 (segment (start 151.20364 87.06612) (end 151.67864 87.06612) (width 0.25) (layer F.Cu) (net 11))
 (segment (start 151.67864 87.06612) (end 153.29516 85.4496) (width 0.25) (layer F.Cu) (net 11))
 (segment (start 153.29516 85.4496) (end 153.29516 81.45228) (width 0.25) (layer F.Cu) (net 11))
 (segment (start 153.29516 81.45228) (end 152.28316 80.44028) (width 0.25) (layer F.Cu) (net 11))
 (segment (start 151.20364 88.33612) (end 152.22864 88.33612) (width 0.25) (layer F.Cu) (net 10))
 (segment (start 152.22864 88.33612) (end 154.82316 85.7416) (width 0.25) (layer F.Cu) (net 10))
 (segment (start 154.82316 85.7416) (end 154.82316 81.45228) (width 0.25) (layer F.Cu) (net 10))
 (segment (start 154.82316 81.45228) (end 154.82316 79.20228) (width 0.25) (layer F.Cu) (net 10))
 (segment (start 151.20364 89.60612) (end 152.22864 89.60612) (width 0.25) (layer F.Cu) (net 9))
 (segment (start 152.22864 89.60612) (end 157.36316 84.4716) (width 0.25) (layer F.Cu) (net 9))
 (segment (start 157.36316 84.4716) (end 157.36316 81.45228) (width 0.25) (layer F.Cu) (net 9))
 (segment (start 157.36316 81.45228) (end 157.36316 79.20228) (width 0.25) (layer F.Cu) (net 9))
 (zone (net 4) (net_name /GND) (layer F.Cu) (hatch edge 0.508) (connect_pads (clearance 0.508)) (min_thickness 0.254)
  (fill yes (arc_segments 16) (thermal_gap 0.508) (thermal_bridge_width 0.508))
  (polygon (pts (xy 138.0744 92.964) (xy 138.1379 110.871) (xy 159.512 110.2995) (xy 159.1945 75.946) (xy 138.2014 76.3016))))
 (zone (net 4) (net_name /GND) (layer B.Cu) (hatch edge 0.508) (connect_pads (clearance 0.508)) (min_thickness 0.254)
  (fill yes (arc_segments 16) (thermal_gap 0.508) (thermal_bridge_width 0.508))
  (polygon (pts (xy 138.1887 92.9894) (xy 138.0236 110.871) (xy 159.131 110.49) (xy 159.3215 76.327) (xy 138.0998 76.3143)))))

